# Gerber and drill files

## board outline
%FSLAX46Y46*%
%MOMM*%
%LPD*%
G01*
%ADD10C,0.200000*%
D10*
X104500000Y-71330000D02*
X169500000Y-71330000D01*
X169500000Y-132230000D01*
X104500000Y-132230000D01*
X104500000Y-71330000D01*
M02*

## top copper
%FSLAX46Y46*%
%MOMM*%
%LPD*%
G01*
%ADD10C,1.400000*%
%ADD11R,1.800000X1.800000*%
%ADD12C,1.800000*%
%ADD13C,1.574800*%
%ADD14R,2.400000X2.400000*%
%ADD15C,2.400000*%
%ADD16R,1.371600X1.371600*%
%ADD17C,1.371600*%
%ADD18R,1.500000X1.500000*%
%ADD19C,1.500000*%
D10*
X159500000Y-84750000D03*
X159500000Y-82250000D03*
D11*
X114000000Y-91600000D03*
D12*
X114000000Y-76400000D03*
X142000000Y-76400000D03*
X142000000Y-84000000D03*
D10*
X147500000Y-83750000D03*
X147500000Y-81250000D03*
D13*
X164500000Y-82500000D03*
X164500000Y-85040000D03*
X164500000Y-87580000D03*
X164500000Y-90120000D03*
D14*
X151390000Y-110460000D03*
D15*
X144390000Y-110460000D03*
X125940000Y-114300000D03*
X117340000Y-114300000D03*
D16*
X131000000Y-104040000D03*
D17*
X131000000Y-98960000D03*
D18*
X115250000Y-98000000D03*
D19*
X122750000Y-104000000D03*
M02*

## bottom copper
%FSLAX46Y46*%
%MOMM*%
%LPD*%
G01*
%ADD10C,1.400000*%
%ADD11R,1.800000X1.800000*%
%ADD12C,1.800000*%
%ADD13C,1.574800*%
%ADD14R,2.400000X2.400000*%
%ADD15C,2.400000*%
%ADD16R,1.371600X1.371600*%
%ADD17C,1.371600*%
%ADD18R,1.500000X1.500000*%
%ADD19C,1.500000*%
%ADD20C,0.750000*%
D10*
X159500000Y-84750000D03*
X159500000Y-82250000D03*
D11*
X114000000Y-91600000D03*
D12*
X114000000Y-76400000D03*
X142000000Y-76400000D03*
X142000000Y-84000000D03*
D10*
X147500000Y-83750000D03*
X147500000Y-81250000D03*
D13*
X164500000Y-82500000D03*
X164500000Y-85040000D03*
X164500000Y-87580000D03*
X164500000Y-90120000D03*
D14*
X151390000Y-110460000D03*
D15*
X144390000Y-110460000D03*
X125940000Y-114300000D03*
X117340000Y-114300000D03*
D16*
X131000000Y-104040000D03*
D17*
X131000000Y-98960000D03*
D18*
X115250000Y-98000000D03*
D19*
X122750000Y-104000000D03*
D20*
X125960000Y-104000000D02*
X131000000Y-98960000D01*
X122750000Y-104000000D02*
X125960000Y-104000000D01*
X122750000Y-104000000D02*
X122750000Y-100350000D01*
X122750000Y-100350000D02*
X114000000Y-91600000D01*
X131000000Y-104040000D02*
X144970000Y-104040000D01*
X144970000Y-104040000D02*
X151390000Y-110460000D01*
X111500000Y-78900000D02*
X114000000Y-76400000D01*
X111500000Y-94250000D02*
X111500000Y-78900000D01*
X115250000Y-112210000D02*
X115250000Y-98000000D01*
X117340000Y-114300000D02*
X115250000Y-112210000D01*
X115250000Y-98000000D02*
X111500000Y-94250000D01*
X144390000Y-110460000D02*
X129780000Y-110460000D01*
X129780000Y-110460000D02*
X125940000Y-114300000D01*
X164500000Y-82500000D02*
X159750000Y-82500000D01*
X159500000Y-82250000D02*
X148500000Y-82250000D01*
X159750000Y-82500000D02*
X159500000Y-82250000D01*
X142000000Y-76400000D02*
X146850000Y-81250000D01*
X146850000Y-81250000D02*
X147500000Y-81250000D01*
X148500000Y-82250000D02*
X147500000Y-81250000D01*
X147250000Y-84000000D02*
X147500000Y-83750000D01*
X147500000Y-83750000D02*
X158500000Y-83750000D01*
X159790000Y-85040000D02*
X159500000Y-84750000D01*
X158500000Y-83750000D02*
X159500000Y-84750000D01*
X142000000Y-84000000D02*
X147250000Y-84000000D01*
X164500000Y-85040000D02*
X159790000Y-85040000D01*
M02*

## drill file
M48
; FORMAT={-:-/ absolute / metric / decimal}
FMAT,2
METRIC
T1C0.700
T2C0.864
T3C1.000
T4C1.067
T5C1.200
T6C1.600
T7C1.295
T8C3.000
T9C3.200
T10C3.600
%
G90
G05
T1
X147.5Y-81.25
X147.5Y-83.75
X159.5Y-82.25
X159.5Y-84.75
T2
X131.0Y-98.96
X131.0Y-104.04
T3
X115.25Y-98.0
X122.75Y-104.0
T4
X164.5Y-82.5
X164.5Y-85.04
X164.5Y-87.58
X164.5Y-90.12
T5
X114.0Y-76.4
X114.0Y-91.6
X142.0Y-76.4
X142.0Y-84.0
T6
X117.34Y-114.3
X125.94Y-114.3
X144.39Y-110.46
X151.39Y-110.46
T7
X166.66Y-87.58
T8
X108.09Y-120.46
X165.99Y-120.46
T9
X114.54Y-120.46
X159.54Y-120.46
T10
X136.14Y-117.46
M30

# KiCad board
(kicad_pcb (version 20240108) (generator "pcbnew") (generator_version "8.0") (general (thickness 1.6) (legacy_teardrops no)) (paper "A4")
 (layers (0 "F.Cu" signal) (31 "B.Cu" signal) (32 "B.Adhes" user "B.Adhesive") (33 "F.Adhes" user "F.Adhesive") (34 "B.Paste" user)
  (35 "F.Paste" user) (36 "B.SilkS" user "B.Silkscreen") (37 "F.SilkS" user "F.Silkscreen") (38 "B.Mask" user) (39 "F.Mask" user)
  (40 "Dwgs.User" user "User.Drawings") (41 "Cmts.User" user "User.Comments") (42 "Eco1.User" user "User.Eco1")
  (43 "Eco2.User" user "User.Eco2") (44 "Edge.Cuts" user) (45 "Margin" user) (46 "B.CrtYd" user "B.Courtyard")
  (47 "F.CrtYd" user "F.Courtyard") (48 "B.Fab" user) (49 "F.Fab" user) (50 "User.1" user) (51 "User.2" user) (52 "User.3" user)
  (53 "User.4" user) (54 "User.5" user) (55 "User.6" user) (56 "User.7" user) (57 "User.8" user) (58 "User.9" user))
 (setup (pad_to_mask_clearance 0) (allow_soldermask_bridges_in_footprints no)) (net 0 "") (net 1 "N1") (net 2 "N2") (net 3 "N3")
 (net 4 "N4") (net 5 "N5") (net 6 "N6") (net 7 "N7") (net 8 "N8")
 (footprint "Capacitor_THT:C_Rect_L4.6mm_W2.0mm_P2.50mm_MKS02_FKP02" (layer "F.Cu") (at 159.5 84.75 90)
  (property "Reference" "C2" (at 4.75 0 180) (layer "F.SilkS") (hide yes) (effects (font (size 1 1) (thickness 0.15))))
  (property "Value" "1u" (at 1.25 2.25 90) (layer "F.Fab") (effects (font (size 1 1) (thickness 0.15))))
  (pad "1" thru_hole circle (at 0 0 90) (size 1.4 1.4) (drill 0.7) (layers "*.Cu" "*.Mask") (remove_unused_layers no) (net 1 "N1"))
  (pad "2" thru_hole circle (at 2.5 0 90) (size 1.4 1.4) (drill 0.7) (layers "*.Cu" "*.Mask") (remove_unused_layers no) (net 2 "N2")))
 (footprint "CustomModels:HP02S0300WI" (layer "F.Cu") (at 114 91.6)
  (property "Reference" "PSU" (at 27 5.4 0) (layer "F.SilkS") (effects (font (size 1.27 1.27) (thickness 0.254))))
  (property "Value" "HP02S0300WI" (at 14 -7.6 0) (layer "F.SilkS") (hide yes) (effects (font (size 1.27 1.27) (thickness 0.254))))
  (pad "1" thru_hole rect (at 0 0) (size 1.8 1.8) (drill 1.2) (layers "*.Cu" "*.Mask") (remove_unused_layers no) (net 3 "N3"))
  (pad "2" thru_hole circle (at 0 -15.2) (size 1.8 1.8) (drill 1.2) (layers "*.Cu" "*.Mask") (remove_unused_layers no) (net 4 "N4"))
  (pad "3" thru_hole circle (at 28 -15.2) (size 1.8 1.8) (drill 1.2) (layers "*.Cu" "*.Mask") (remove_unused_layers no) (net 2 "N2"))
  (pad "4" thru_hole circle (at 28 -7.6) (size 1.8 1.8) (drill 1.2) (layers "*.Cu" "*.Mask") (remove_unused_layers no) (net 1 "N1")))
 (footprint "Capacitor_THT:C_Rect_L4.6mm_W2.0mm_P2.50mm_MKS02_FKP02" (layer "F.Cu") (at 147.5 83.75 90)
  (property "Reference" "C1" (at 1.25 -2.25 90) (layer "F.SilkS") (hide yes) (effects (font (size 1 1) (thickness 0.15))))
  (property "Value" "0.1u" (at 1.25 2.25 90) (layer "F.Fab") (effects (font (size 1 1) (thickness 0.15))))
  (pad "1" thru_hole circle (at 0 0 90) (size 1.4 1.4) (drill 0.7) (layers "*.Cu" "*.Mask") (remove_unused_layers no) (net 1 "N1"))
  (pad "2" thru_hole circle (at 2.5 0 90) (size 1.4 1.4) (drill 0.7) (layers "*.Cu" "*.Mask") (remove_unused_layers no) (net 2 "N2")))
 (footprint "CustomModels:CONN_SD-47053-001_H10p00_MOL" (layer "F.Cu") (at 164.5 82.5 90)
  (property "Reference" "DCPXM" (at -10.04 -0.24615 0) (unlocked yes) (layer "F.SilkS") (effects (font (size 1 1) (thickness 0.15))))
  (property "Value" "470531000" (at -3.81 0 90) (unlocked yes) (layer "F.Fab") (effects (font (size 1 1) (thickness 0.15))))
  (pad "" np_thru_hole circle (at -5.08 2.16 90) (size 1.2954 1.2954) (drill 1.2954) (layers "*.SilkS"))
  (pad "1" thru_hole circle (at 0 0 90) (size 1.5748 1.5748) (drill 1.0668) (layers "*.Cu" "*.Mask") (remove_unused_layers no) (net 2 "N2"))
  (pad "2" thru_hole circle (at -2.54 0 90) (size 1.5748 1.5748) (drill 1.0668) (layers "*.Cu" "*.Mask") (remove_unused_layers no)
   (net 1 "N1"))
  (pad "3" thru_hole circle (at -5.08 0 90) (size 1.5748 1.5748) (drill 1.0668) (layers "*.Cu" "*.Mask") (remove_unused_layers no)
   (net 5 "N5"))
  (pad "4" thru_hole circle (at -7.62 0 90) (size 1.5748 1.5748) (drill 1.0668) (layers "*.Cu" "*.Mask") (remove_unused_layers no)
   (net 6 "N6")))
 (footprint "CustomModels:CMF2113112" (layer "F.Cu") (at 151.39 110.46)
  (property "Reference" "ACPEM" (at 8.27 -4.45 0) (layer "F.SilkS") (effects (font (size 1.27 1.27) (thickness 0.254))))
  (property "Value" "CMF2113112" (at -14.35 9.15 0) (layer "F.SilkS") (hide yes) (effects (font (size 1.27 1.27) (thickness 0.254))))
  (pad "" np_thru_hole circle (at -43.3 10) (size 3 3) (drill 3) (layers "*.SilkS"))
  (pad "" np_thru_hole circle (at -36.85 10) (size 3.2 3.2) (drill 3.2) (layers "*.SilkS"))
  (pad "" np_thru_hole circle (at -15.25 7) (size 3.6 3.6) (drill 3.6) (layers "*.SilkS"))
  (pad "" np_thru_hole circle (at 8.15 10) (size 3.2 3.2) (drill 3.2) (layers "*.SilkS"))
  (pad "" np_thru_hole circle (at 14.6 10) (size 3 3) (drill 3) (layers "*.SilkS"))
  (pad "1" thru_hole rect (at 0 0) (size 2.4 2.4) (drill 1.6) (layers "*.Cu" "*.Mask") (remove_unused_layers no) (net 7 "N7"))
  (pad "2" thru_hole circle (at -7 0) (size 2.4 2.4) (drill 1.6) (layers "*.Cu" "*.Mask") (remove_unused_layers no) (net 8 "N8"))
  (pad "L1" thru_hole circle (at -25.45 3.84) (size 2.4 2.4) (drill 1.6) (layers "*.Cu" "*.Mask") (remove_unused_layers no) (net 8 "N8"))
  (pad "N1" thru_hole circle (at -34.05 3.84) (size 2.4 2.4) (drill 1.6) (layers "*.Cu" "*.Mask") (remove_unused_layers no) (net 4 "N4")))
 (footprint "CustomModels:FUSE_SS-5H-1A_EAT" (layer "F.Cu") (at 131 104.04 90)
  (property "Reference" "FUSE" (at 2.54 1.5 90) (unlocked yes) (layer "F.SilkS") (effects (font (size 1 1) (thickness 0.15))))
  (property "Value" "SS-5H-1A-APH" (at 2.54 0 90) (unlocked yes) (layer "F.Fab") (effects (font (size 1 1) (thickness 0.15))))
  (pad "1" thru_hole rect (at 0 0 90) (size 1.3716 1.3716) (drill 0.8636) (layers "*.Cu" "*.Mask") (remove_unused_layers no) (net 7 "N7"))
  (pad "2" thru_hole circle (at 5.08 0 90) (size 1.3716 1.3716) (drill 0.8636) (layers "*.Cu" "*.Mask") (remove_unused_layers no)
   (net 3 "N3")))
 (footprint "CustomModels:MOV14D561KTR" (layer "F.Cu") (at 115.25 98)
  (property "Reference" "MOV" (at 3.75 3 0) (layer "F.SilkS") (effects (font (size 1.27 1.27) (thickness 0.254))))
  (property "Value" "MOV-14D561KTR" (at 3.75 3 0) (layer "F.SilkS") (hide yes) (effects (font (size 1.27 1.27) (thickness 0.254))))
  (pad "1" thru_hole rect (at 0 0) (size 1.5 1.5) (drill 1) (layers "*.Cu" "*.Mask") (remove_unused_layers no) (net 4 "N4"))
  (pad "2" thru_hole circle (at 7.5 6) (size 1.5 1.5) (drill 1) (layers "*.Cu" "*.Mask") (remove_unused_layers no) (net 3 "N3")))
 (gr_rect (start 104.5 71.33) (end 169.5 132.23) (stroke (width 0.2) (type default)) (fill none) (layer "Edge.Cuts"))
 (segment (start 125.96 104) (end 131 98.96) (width 0.75) (layer "B.Cu") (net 3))
 (segment (start 122.75 104) (end 125.96 104) (width 0.75) (layer "B.Cu") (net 3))
 (segment (start 122.75 104) (end 122.75 100.35) (width 0.75) (layer "B.Cu") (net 3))
 (segment (start 122.75 100.35) (end 114 91.6) (width 0.75) (layer "B.Cu") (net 3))
 (segment (start 131 104.04) (end 144.97 104.04) (width 0.75) (layer "B.Cu") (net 7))
 (segment (start 144.97 104.04) (end 151.39 110.46) (width 0.75) (layer "B.Cu") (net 7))
 (segment (start 111.5 78.9) (end 114 76.4) (width 0.75) (layer "B.Cu") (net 4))
 (segment (start 111.5 94.25) (end 111.5 78.9) (width 0.75) (layer "B.Cu") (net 4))
 (segment (start 115.25 112.21) (end 115.25 98) (width 0.75) (layer "B.Cu") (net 4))
 (segment (start 117.34 114.3) (end 115.25 112.21) (width 0.75) (layer "B.Cu") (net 4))
 (segment (start 115.25 98) (end 111.5 94.25) (width 0.75) (layer "B.Cu") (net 4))
 (segment (start 144.39 110.46) (end 129.78 110.46) (width 0.75) (layer "B.Cu") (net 8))
 (segment (start 129.78 110.46) (end 125.94 114.3) (width 0.75) (layer "B.Cu") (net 8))
 (segment (start 164.5 82.5) (end 159.75 82.5) (width 0.75) (layer "B.Cu") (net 2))
 (segment (start 159.5 82.25) (end 148.5 82.25) (width 0.75) (layer "B.Cu") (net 2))
 (segment (start 159.75 82.5) (end 159.5 82.25) (width 0.75) (layer "B.Cu") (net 2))
 (segment (start 142 76.4) (end 146.85 81.25) (width 0.75) (layer "B.Cu") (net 2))
 (segment (start 146.85 81.25) (end 147.5 81.25) (width 0.75) (layer "B.Cu") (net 2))
 (segment (start 148.5 82.25) (end 147.5 81.25) (width 0.75) (layer "B.Cu") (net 2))
 (segment (start 147.25 84) (end 147.5 83.75) (width 0.75) (layer "B.Cu") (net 1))
 (segment (start 147.5 83.75) (end 158.5 83.75) (width 0.75) (layer "B.Cu") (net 1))
 (segment (start 159.79 85.04) (end 159.5 84.75) (width 0.75) (layer "B.Cu") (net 1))
 (segment (start 158.5 83.75) (end 159.5 84.75) (width 0.75) (layer "B.Cu") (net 1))
 (segment (start 142 84) (end 147.25 84) (width 0.75) (layer "B.Cu") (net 1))
 (segment (start 164.5 85.04) (end 159.79 85.04) (width 0.75) (layer "B.Cu") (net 1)))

